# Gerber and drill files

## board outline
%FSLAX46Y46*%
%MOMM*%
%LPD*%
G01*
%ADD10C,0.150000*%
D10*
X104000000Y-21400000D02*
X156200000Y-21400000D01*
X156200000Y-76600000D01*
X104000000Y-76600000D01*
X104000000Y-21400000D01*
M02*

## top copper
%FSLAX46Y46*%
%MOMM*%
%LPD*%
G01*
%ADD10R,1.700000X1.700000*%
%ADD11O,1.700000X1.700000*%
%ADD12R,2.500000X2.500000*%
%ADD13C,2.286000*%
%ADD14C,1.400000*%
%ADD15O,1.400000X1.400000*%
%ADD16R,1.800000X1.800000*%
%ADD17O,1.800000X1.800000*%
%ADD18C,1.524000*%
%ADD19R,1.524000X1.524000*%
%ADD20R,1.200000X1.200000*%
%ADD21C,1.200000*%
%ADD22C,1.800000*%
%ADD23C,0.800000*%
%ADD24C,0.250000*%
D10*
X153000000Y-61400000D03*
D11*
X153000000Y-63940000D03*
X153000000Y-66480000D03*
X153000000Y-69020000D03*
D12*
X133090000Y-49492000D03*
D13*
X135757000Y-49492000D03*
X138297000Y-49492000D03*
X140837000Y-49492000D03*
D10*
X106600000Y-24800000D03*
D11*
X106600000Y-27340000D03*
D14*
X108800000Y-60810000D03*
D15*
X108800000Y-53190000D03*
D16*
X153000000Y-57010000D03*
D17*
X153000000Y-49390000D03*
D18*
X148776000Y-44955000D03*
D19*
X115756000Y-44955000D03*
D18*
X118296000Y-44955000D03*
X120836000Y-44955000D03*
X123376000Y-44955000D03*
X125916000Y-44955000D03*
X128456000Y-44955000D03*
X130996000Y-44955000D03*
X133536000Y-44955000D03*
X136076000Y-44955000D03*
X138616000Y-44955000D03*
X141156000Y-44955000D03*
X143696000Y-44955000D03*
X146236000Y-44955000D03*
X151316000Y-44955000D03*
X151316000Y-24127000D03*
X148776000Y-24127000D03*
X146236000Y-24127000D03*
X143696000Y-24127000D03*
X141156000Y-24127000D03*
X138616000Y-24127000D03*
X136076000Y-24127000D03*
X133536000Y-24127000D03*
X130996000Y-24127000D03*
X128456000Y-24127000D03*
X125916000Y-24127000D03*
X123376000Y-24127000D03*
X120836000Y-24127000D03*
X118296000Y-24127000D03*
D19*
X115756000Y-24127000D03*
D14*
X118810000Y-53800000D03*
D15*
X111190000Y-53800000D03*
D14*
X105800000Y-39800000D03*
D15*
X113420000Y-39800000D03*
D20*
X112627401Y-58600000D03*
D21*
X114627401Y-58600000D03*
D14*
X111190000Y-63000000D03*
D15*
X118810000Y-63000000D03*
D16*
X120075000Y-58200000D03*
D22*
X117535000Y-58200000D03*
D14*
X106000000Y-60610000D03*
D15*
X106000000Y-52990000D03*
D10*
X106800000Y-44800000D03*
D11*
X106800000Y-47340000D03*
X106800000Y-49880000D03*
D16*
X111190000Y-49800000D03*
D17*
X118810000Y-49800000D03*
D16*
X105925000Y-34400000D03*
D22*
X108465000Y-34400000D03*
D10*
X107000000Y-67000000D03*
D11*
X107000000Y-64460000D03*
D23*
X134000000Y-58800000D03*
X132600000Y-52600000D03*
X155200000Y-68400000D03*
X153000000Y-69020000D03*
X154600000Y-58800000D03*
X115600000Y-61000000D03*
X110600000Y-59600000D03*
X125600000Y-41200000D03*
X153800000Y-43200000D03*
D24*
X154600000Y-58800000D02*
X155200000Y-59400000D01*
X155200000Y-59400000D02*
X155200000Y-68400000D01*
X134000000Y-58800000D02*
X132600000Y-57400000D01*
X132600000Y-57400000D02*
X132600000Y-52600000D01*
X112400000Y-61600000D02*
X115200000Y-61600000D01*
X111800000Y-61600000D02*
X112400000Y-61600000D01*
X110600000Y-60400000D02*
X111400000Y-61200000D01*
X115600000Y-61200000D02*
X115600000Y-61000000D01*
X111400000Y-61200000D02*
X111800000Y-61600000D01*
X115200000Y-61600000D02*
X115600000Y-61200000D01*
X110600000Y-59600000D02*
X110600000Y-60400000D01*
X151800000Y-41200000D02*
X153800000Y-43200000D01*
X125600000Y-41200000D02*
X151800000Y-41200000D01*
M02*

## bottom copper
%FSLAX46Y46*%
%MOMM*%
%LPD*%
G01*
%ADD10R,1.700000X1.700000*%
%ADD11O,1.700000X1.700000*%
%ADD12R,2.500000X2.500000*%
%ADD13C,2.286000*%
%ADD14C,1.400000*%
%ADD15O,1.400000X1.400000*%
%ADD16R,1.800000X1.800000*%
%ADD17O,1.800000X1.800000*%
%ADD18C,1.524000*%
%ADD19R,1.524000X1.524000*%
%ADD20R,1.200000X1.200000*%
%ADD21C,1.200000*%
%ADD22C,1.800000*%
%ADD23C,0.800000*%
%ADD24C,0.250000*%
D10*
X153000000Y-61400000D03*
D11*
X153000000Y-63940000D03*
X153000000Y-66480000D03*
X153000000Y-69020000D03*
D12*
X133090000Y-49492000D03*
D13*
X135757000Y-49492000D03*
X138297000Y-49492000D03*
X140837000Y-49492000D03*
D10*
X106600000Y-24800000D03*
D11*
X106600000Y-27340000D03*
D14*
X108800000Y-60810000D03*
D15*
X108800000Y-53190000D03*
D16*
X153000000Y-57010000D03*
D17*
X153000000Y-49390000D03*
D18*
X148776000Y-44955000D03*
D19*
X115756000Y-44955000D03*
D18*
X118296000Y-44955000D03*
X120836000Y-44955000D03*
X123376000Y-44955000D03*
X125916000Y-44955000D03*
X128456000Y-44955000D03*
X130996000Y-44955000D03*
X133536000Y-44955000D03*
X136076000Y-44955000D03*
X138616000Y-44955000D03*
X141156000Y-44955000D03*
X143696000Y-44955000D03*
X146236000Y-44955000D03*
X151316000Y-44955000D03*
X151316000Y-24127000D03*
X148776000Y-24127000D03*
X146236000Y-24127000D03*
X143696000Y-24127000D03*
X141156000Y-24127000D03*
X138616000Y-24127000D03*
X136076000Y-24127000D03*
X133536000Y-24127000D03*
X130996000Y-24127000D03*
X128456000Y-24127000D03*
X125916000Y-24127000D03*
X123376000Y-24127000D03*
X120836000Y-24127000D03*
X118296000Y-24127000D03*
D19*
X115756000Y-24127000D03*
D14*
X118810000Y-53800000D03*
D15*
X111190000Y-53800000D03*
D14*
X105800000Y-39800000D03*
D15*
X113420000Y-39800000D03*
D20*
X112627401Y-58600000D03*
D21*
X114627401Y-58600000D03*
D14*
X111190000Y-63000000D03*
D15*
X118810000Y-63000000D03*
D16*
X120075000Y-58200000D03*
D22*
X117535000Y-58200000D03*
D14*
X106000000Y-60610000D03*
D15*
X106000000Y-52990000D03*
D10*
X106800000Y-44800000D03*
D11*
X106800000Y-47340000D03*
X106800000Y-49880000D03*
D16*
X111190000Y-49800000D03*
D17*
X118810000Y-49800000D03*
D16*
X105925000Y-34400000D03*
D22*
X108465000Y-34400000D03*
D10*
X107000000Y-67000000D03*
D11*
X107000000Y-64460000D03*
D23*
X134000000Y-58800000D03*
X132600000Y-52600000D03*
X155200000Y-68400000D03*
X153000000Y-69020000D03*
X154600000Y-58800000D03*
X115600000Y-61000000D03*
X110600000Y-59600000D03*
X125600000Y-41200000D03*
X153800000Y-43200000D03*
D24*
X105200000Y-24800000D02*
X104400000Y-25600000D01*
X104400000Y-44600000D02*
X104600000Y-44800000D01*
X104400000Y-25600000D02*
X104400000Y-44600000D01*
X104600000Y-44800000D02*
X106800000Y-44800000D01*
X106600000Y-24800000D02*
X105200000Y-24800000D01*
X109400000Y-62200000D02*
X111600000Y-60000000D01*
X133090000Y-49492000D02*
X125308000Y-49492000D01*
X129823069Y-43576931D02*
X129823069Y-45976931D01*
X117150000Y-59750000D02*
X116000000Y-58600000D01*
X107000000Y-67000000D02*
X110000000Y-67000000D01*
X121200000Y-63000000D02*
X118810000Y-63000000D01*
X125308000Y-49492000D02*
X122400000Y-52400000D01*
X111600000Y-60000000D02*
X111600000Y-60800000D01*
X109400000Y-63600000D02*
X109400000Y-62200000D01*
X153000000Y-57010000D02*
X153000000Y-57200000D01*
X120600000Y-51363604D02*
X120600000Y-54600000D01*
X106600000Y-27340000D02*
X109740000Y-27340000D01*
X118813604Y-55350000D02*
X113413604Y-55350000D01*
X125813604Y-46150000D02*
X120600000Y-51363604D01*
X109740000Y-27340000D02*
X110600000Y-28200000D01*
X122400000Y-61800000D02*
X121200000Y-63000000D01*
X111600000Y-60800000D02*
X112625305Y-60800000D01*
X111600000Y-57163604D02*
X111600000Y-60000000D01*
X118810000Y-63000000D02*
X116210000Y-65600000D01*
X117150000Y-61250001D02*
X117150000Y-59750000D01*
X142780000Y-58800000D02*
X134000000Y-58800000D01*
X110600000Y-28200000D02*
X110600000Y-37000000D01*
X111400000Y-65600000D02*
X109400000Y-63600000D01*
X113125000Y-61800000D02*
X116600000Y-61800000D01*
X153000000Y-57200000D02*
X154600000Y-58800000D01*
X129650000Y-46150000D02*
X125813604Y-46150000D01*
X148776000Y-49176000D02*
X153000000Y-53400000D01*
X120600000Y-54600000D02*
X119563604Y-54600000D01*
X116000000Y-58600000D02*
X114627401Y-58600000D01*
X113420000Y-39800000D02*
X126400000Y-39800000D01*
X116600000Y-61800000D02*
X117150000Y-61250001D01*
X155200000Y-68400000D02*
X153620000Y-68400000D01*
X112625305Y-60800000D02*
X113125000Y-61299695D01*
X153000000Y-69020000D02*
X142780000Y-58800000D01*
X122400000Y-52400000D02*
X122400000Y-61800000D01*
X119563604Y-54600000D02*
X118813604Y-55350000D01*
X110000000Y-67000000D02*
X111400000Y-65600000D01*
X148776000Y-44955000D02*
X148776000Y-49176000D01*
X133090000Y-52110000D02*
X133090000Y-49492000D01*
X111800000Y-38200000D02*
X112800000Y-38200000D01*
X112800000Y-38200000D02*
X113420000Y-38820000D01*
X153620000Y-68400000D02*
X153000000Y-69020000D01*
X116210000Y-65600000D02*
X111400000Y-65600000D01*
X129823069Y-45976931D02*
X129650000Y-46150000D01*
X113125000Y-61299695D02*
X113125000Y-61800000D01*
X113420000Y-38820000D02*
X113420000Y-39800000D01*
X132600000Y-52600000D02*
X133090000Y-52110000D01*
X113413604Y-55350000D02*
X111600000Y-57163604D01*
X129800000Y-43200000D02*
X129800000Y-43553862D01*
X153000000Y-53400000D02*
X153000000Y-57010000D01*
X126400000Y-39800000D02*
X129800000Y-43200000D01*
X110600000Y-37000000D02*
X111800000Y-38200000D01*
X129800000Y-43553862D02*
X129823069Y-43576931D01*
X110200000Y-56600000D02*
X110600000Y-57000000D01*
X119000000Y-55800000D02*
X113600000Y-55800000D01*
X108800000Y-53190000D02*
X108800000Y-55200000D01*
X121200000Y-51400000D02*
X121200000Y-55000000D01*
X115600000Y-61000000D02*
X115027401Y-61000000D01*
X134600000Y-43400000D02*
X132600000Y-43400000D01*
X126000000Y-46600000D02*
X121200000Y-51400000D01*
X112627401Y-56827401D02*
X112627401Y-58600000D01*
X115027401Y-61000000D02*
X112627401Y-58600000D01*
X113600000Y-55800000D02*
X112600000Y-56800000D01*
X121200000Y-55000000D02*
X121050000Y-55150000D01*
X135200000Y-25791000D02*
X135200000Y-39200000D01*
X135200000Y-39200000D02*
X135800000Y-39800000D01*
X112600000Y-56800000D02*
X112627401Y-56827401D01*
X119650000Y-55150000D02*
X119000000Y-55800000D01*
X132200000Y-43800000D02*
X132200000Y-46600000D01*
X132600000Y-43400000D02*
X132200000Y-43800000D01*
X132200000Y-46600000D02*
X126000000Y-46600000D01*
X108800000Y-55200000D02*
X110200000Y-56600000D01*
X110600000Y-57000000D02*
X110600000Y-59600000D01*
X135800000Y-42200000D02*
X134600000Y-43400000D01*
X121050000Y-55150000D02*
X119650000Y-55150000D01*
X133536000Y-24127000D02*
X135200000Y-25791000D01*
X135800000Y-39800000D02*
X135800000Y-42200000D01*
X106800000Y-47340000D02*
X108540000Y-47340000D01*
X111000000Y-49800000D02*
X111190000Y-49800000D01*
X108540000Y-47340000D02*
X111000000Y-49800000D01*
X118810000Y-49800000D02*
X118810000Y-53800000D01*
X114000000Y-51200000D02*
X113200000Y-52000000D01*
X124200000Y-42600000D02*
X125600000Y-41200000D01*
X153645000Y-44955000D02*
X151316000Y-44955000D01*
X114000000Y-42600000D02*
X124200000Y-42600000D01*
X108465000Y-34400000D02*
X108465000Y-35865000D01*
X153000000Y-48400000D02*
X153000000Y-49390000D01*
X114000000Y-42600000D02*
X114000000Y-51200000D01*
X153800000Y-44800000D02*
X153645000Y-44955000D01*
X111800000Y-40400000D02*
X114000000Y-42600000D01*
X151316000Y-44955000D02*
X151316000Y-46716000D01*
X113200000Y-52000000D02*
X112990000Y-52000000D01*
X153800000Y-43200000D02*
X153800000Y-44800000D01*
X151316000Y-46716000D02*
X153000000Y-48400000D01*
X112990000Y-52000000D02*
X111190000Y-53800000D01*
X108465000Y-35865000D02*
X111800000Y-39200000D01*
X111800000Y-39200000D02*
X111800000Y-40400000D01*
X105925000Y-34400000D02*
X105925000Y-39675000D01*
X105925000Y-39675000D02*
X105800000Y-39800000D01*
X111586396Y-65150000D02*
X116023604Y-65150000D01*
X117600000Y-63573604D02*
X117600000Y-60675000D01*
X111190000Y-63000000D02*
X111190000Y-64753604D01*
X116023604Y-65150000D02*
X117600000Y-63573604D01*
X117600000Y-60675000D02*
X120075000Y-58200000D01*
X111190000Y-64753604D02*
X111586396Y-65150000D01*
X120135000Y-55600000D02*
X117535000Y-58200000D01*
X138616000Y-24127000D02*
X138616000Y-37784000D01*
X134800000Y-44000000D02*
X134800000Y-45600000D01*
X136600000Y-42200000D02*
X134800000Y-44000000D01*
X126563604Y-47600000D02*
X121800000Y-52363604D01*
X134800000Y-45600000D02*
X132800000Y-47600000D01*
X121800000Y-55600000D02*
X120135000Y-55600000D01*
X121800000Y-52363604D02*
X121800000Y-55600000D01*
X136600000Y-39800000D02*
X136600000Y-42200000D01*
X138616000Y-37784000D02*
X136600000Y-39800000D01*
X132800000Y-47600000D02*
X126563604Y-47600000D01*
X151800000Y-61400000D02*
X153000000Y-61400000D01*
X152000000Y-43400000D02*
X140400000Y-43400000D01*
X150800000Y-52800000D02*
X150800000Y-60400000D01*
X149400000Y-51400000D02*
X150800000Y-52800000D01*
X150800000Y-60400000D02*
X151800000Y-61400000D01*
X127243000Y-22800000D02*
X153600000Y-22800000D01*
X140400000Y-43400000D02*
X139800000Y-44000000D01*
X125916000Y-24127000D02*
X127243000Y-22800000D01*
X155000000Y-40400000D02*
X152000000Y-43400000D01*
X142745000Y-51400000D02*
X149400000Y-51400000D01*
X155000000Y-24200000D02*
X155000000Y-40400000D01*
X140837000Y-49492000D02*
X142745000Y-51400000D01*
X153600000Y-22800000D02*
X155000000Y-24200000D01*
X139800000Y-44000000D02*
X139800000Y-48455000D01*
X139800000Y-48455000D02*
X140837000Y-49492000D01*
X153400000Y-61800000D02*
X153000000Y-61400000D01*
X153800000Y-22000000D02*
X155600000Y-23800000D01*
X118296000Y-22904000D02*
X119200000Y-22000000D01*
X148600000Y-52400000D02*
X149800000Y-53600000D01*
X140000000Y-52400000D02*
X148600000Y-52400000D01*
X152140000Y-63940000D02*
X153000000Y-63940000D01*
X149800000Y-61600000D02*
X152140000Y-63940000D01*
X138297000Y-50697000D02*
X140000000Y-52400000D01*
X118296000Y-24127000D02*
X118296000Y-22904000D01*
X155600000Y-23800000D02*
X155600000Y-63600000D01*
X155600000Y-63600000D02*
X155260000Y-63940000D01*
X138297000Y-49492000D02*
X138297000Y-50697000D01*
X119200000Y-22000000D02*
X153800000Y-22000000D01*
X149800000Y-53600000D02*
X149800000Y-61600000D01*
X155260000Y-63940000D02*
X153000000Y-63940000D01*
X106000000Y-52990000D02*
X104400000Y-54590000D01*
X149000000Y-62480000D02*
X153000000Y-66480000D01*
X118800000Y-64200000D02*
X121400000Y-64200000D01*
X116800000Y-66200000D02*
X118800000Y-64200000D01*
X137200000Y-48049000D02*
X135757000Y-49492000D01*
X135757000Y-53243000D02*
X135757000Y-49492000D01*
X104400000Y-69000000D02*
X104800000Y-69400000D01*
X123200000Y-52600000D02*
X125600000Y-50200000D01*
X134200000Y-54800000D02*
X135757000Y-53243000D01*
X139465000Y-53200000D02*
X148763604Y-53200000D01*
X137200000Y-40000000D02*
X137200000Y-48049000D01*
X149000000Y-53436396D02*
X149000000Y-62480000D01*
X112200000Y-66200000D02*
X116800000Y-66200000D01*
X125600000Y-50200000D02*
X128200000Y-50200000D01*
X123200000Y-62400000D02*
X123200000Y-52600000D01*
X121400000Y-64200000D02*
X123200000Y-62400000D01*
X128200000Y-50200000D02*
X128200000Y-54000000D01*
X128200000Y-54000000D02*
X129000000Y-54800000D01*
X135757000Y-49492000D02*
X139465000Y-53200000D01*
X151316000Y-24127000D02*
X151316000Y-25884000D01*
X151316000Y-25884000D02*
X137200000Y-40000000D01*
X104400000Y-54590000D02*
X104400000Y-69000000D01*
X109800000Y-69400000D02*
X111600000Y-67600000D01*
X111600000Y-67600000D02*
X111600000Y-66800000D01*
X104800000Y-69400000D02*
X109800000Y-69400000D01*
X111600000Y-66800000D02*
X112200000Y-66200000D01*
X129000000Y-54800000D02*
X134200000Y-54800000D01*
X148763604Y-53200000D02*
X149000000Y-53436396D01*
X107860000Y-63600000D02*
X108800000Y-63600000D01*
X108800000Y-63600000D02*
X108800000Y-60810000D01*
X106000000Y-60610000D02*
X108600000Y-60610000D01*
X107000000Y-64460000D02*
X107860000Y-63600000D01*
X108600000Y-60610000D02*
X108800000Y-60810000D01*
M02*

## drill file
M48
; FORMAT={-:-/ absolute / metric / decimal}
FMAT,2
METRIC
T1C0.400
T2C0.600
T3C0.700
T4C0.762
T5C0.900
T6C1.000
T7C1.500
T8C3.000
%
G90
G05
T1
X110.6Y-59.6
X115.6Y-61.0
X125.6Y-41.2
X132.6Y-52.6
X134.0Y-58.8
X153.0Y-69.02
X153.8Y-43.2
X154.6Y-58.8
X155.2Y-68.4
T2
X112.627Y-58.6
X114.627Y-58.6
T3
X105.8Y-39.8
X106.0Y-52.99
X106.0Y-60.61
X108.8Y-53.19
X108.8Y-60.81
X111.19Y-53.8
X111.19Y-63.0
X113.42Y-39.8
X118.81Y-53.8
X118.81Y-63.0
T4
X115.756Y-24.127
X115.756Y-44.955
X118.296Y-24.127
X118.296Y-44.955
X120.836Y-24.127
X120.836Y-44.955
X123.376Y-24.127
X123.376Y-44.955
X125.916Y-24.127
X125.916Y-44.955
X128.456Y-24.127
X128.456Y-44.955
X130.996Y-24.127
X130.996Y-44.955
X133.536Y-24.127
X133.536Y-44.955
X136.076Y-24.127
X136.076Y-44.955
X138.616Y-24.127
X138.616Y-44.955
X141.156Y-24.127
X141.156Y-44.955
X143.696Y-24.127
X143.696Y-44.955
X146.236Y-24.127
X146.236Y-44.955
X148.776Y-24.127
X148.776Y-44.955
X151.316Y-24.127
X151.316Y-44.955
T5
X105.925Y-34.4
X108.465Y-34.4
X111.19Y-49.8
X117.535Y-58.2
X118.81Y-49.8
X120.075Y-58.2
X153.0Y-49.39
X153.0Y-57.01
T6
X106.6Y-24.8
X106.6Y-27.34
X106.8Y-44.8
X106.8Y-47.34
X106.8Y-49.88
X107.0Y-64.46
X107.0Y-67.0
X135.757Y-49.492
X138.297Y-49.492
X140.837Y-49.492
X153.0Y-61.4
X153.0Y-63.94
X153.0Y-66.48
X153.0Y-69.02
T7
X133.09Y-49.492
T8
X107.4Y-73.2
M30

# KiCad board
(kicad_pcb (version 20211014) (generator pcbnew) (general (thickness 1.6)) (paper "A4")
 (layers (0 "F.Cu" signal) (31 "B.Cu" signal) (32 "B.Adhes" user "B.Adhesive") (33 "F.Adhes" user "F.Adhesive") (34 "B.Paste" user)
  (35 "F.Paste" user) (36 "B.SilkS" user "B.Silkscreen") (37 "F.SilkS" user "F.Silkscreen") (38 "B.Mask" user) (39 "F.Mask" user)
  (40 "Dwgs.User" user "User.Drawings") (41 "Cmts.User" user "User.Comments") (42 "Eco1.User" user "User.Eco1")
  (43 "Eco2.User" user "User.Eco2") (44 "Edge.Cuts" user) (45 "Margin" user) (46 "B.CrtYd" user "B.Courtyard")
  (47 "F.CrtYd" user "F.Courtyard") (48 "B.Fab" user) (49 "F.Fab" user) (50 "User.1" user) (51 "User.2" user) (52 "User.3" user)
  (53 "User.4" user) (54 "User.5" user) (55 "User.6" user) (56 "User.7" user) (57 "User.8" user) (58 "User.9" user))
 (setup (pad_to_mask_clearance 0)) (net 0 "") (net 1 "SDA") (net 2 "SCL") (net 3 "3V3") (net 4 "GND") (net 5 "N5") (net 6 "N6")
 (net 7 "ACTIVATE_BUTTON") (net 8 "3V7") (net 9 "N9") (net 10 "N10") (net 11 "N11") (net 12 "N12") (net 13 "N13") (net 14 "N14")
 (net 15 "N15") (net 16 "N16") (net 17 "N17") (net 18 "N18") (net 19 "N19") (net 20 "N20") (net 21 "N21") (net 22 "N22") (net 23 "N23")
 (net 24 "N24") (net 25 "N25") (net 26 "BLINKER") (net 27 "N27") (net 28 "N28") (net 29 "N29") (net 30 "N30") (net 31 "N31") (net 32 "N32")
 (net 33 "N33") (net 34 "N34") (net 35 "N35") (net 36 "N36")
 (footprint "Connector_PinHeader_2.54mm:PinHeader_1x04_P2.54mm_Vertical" (layer "F.Cu") (at 153 61.4)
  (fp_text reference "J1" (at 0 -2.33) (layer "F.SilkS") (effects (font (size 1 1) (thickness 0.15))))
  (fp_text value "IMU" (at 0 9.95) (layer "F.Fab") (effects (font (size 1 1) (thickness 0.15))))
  (pad "1" thru_hole rect (at 0 0) (size 1.7 1.7) (drill 1) (layers *.Cu *.Mask) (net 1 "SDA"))
  (pad "2" thru_hole oval (at 0 2.54) (size 1.7 1.7) (drill 1) (layers *.Cu *.Mask) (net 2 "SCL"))
  (pad "3" thru_hole oval (at 0 5.08) (size 1.7 1.7) (drill 1) (layers *.Cu *.Mask) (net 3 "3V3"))
  (pad "4" thru_hole oval (at 0 7.62) (size 1.7 1.7) (drill 1) (layers *.Cu *.Mask) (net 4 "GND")))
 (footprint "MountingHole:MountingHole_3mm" (layer "F.Cu") (at 107.4 73.2)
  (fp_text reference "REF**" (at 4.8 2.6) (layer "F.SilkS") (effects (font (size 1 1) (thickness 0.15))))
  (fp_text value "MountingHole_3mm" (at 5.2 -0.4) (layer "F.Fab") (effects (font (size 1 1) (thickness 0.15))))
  (pad "" np_thru_hole circle (at 0 0) (size 3 3) (drill 3) (layers *.Cu *.Mask)))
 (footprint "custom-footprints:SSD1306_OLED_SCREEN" (layer "F.Cu") (at 122.295 48.095)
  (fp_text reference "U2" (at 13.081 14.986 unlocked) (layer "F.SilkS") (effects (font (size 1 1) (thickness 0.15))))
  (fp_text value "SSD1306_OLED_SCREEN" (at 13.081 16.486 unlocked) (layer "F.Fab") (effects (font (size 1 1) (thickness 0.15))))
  (pad "1" thru_hole rect (at 10.795 1.397) (size 2.5 2.5) (drill 1.5) (layers *.Cu *.Mask) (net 4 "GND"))
  (pad "2" thru_hole circle (at 13.462 1.397) (size 2.286 2.286) (drill 1) (layers *.Cu *.Mask) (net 3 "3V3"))
  (pad "3" thru_hole circle (at 16.002 1.397) (size 2.286 2.286) (drill 1) (layers *.Cu *.Mask) (remove_unused_layers) (keep_end_layers)
   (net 2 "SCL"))
  (pad "4" thru_hole circle (at 18.542 1.397) (size 2.286 2.286) (drill 1) (layers *.Cu *.Mask) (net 1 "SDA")))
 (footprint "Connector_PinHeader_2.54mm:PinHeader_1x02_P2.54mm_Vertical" (layer "F.Cu") (at 106.6 24.8)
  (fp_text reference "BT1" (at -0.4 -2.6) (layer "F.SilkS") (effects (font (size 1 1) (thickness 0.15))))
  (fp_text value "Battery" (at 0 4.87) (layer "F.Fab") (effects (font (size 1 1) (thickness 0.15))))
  (pad "1" thru_hole rect (at 0 0) (size 1.7 1.7) (drill 1) (layers *.Cu *.Mask) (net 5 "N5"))
  (pad "2" thru_hole oval (at 0 2.54) (size 1.7 1.7) (drill 1) (layers *.Cu *.Mask) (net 4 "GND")))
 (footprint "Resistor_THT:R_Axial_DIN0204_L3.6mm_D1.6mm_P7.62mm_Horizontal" (layer "F.Cu") (at 108.8 60.81 90)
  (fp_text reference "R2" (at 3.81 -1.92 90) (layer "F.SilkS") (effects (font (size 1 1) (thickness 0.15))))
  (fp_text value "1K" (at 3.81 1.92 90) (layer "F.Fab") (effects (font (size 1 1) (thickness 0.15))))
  (pad "1" thru_hole circle (at 0 0 90) (size 1.4 1.4) (drill 0.7) (layers *.Cu *.Mask) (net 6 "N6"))
  (pad "2" thru_hole oval (at 7.62 0 90) (size 1.4 1.4) (drill 0.7) (layers *.Cu *.Mask) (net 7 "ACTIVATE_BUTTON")))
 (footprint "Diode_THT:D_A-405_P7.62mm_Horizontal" (layer "F.Cu") (at 153 57.01 90)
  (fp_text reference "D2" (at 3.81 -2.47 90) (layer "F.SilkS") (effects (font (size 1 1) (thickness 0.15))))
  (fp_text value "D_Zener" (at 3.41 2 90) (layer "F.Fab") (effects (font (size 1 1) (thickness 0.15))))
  (pad "1" thru_hole rect (at 0 0 90) (size 1.8 1.8) (drill 0.9) (layers *.Cu *.Mask) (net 4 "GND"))
  (pad "2" thru_hole oval (at 7.62 0 90) (size 1.8 1.8) (drill 0.9) (layers *.Cu *.Mask) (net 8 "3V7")))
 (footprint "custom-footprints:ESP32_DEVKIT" (layer "F.Cu") (at 110.295 46.225 90)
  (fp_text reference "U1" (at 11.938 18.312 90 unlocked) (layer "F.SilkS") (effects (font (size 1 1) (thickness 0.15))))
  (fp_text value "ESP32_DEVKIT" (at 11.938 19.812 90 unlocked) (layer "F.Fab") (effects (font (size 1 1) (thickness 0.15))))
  (pad "1" thru_hole circle (at 1.27 38.481 90) (size 1.524 1.524) (drill 0.762) (layers *.Cu *.Mask) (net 4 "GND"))
  (pad "2" thru_hole rect (at 1.27 5.461 90) (size 1.524 1.524) (drill oval 0.762) (layers *.Cu *.Mask) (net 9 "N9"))
  (pad "3" thru_hole circle (at 1.27 8.001 90) (size 1.524 1.524) (drill 0.762) (layers *.Cu *.Mask) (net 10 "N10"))
  (pad "4" thru_hole circle (at 1.27 10.541 90) (size 1.524 1.524) (drill 0.762) (layers *.Cu *.Mask) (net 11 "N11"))
  (pad "5" thru_hole circle (at 1.27 13.081 90) (size 1.524 1.524) (drill 0.762) (layers *.Cu *.Mask) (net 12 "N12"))
  (pad "6" thru_hole circle (at 1.27 15.621 90) (size 1.524 1.524) (drill 0.762) (layers *.Cu *.Mask) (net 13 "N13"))
  (pad "7" thru_hole circle (at 1.27 18.161 90) (size 1.524 1.524) (drill 0.762) (layers *.Cu *.Mask) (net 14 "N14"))
  (pad "8" thru_hole circle (at 1.27 20.701 90) (size 1.524 1.524) (drill 0.762) (layers *.Cu *.Mask) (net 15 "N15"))
  (pad "9" thru_hole circle (at 1.27 23.241 90) (size 1.524 1.524) (drill 0.762) (layers *.Cu *.Mask) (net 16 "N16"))
  (pad "10" thru_hole circle (at 1.27 25.781 90) (size 1.524 1.524) (drill 0.762) (layers *.Cu *.Mask) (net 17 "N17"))
  (pad "11" thru_hole circle (at 1.27 28.321 90) (size 1.524 1.524) (drill 0.762) (layers *.Cu *.Mask) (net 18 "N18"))
  (pad "12" thru_hole circle (at 1.27 30.861 90) (size 1.524 1.524) (drill 0.762) (layers *.Cu *.Mask) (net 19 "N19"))
  (pad "13" thru_hole circle (at 1.27 33.401 90) (size 1.524 1.524) (drill 0.762) (layers *.Cu *.Mask) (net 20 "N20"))
  (pad "14" thru_hole circle (at 1.27 35.941 90) (size 1.524 1.524) (drill 0.762) (layers *.Cu *.Mask) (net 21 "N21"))
  (pad "16" thru_hole circle (at 1.27 41.021 90) (size 1.524 1.524) (drill 0.762) (layers *.Cu *.Mask) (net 8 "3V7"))
  (pad "24" thru_hole circle (at 22.098 41.021 90) (size 1.524 1.524) (drill 0.762) (layers *.Cu *.Mask) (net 3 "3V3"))
  (pad "25" thru_hole circle (at 22.098 38.481 90) (size 1.524 1.524) (drill 0.762) (layers *.Cu *.Mask) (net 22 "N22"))
  (pad "26" thru_hole circle (at 22.098 35.941 90) (size 1.524 1.524) (drill 0.762) (layers *.Cu *.Mask) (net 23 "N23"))
  (pad "27" thru_hole circle (at 22.098 33.401 90) (size 1.524 1.524) (drill 0.762) (layers *.Cu *.Mask) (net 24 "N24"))
  (pad "28" thru_hole circle (at 22.098 30.861 90) (size 1.524 1.524) (drill 0.762) (layers *.Cu *.Mask) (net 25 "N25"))
  (pad "29" thru_hole circle (at 22.098 28.321 90) (size 1.524 1.524) (drill 0.762) (layers *.Cu *.Mask) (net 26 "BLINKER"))
  (pad "30" thru_hole circle (at 22.098 25.781 90) (size 1.524 1.524) (drill 0.762) (layers *.Cu *.Mask) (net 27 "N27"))
  (pad "31" thru_hole circle (at 22.098 23.241 90) (size 1.524 1.524) (drill 0.762) (layers *.Cu *.Mask) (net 7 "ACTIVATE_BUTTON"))
  (pad "32" thru_hole circle (at 22.098 20.701 90) (size 1.524 1.524) (drill 0.762) (layers *.Cu *.Mask) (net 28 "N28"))
  (pad "33" thru_hole circle (at 22.098 18.161 90) (size 1.524 1.524) (drill 0.762) (layers *.Cu *.Mask) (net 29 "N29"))
  (pad "34" thru_hole circle (at 22.098 15.621 90) (size 1.524 1.524) (drill 0.762) (layers *.Cu *.Mask) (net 1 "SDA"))
  (pad "35" thru_hole circle (at 22.098 13.081 90) (size 1.524 1.524) (drill 0.762) (layers *.Cu *.Mask) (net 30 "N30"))
  (pad "36" thru_hole circle (at 22.098 10.541 90) (size 1.524 1.524) (drill 0.762) (layers *.Cu *.Mask) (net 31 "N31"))
  (pad "37" thru_hole circle (at 22.098 8.001 90) (size 1.524 1.524) (drill 0.762) (layers *.Cu *.Mask) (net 2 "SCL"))
  (pad "38" thru_hole rect (at 22.098 5.461 90) (size 1.524 1.524) (drill 0.762) (layers *.Cu *.Mask) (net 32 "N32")))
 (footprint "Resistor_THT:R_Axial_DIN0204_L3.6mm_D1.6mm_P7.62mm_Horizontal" (layer "F.Cu") (at 118.81 53.8 180)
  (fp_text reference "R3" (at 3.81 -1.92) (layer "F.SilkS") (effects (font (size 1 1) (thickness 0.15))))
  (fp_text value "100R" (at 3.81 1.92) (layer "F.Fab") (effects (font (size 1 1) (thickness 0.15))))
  (pad "1" thru_hole circle (at 0 0 180) (size 1.4 1.4) (drill 0.7) (layers *.Cu *.Mask) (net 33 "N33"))
  (pad "2" thru_hole oval (at 7.62 0 180) (size 1.4 1.4) (drill 0.7) (layers *.Cu *.Mask) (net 8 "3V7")))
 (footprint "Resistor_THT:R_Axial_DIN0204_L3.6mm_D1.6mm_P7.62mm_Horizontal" (layer "F.Cu") (at 105.8 39.8)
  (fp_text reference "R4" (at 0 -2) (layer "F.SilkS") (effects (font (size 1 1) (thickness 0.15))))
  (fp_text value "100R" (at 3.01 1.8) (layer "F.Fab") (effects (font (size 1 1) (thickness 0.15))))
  (pad "1" thru_hole circle (at 0 0) (size 1.4 1.4) (drill 0.7) (layers *.Cu *.Mask) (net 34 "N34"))
  (pad "2" thru_hole oval (at 7.62 0) (size 1.4 1.4) (drill 0.7) (layers *.Cu *.Mask) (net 4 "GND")))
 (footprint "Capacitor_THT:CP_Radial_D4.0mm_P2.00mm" (layer "F.Cu") (at 112.627401 58.6)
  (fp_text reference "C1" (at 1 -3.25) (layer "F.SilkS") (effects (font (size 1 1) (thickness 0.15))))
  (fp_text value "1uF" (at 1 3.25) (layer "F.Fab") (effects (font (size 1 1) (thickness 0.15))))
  (pad "1" thru_hole rect (at 0 0) (size 1.2 1.2) (drill 0.6) (layers *.Cu *.Mask) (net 7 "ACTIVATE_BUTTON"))
  (pad "2" thru_hole circle (at 2 0) (size 1.2 1.2) (drill 0.6) (layers *.Cu *.Mask) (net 4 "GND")))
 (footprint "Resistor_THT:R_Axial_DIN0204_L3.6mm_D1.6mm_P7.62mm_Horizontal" (layer "F.Cu") (at 111.19 63)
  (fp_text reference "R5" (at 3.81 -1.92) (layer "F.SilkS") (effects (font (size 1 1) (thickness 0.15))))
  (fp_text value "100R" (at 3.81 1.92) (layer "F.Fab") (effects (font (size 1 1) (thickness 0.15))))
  (pad "1" thru_hole circle (at 0 0) (size 1.4 1.4) (drill 0.7) (layers *.Cu *.Mask) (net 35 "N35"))
  (pad "2" thru_hole oval (at 7.62 0) (size 1.4 1.4) (drill 0.7) (layers *.Cu *.Mask) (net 4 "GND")))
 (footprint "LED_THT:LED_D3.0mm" (layer "F.Cu") (at 120.075 58.2 180)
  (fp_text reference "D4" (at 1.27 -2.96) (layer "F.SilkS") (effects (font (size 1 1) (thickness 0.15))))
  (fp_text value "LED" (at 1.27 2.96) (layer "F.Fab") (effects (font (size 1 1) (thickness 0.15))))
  (pad "1" thru_hole rect (at 0 0 180) (size 1.8 1.8) (drill 0.9) (layers *.Cu *.Mask) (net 35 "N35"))
  (pad "2" thru_hole circle (at 2.54 0 180) (size 1.8 1.8) (drill 0.9) (layers *.Cu *.Mask) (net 26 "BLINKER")))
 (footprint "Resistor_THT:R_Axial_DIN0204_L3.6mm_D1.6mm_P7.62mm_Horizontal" (layer "F.Cu") (at 106 60.61 90)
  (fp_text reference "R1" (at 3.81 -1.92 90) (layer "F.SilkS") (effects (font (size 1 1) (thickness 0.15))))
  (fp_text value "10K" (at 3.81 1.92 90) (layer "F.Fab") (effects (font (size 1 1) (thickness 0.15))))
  (pad "1" thru_hole circle (at 0 0 90) (size 1.4 1.4) (drill 0.7) (layers *.Cu *.Mask) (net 6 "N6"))
  (pad "2" thru_hole oval (at 7.62 0 90) (size 1.4 1.4) (drill 0.7) (layers *.Cu *.Mask) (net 3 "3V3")))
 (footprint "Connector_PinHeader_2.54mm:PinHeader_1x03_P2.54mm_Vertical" (layer "F.Cu") (at 106.8 44.8)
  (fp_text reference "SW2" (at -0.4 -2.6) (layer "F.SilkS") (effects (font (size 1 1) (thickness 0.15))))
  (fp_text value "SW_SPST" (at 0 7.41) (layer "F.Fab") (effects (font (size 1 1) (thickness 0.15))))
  (pad "1" thru_hole rect (at 0 0) (size 1.7 1.7) (drill 1) (layers *.Cu *.Mask) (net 5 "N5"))
  (pad "2" thru_hole oval (at 0 2.54) (size 1.7 1.7) (drill 1) (layers *.Cu *.Mask) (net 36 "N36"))
  (pad "3" thru_hole oval (at 0 5.08) (size 1.7 1.7) (drill 1) (layers *.Cu *.Mask)))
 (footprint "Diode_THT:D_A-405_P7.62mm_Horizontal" (layer "F.Cu") (at 111.19 49.8)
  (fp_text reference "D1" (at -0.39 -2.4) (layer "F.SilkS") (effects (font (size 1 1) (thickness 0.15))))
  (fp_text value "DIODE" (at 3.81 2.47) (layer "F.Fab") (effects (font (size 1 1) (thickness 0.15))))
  (pad "1" thru_hole rect (at 0 0) (size 1.8 1.8) (drill 0.9) (layers *.Cu *.Mask) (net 36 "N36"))
  (pad "2" thru_hole oval (at 7.62 0) (size 1.8 1.8) (drill 0.9) (layers *.Cu *.Mask) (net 33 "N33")))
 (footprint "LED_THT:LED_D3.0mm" (layer "F.Cu") (at 105.925 34.4)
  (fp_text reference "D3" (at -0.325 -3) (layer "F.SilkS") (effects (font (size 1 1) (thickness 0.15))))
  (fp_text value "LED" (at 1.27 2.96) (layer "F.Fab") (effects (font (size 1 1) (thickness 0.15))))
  (pad "1" thru_hole rect (at 0 0) (size 1.8 1.8) (drill 0.9) (layers *.Cu *.Mask) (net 34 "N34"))
  (pad "2" thru_hole circle (at 2.54 0) (size 1.8 1.8) (drill 0.9) (layers *.Cu *.Mask) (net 8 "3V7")))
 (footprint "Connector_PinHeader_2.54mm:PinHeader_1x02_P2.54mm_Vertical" (layer "F.Cu") (at 107 67 180)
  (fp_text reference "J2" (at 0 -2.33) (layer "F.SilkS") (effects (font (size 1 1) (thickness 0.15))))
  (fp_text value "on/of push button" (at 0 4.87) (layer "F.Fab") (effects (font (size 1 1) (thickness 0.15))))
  (pad "1" thru_hole rect (at 0 0 180) (size 1.7 1.7) (drill 1) (layers *.Cu *.Mask) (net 4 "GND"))
  (pad "2" thru_hole oval (at 0 2.54 180) (size 1.7 1.7) (drill 1) (layers *.Cu *.Mask) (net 6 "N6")))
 (gr_rect (start 104 21.4) (end 156.2 76.6) (layer "Edge.Cuts") (width 0.15) (fill none))
 (segment (start 105.2 24.8) (end 104.4 25.6) (width 0.25) (layer "B.Cu") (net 5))
 (segment (start 104.4 44.6) (end 104.6 44.8) (width 0.25) (layer "B.Cu") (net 5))
 (segment (start 104.4 25.6) (end 104.4 44.6) (width 0.25) (layer "B.Cu") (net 5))
 (segment (start 104.6 44.8) (end 106.8 44.8) (width 0.25) (layer "B.Cu") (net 5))
 (segment (start 106.6 24.8) (end 105.2 24.8) (width 0.25) (layer "B.Cu") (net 5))
 (segment (start 154.6 58.8) (end 155.2 59.4) (width 0.25) (layer "F.Cu") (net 4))
 (segment (start 155.2 59.4) (end 155.2 68.4) (width 0.25) (layer "F.Cu") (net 4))
 (segment (start 134 58.8) (end 132.6 57.4) (width 0.25) (layer "F.Cu") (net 4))
 (segment (start 132.6 57.4) (end 132.6 52.6) (width 0.25) (layer "F.Cu") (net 4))
 (via (at 134 58.8) (size 0.8) (drill 0.4) (layers "F.Cu" "B.Cu") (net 4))
 (via (at 132.6 52.6) (size 0.8) (drill 0.4) (layers "F.Cu" "B.Cu") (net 4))
 (via (at 155.2 68.4) (size 0.8) (drill 0.4) (layers "F.Cu" "B.Cu") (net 4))
 (via (at 153 69.02) (size 0.8) (drill 0.4) (layers "F.Cu" "B.Cu") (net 4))
 (via (at 154.6 58.8) (size 0.8) (drill 0.4) (layers "F.Cu" "B.Cu") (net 4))
 (segment (start 109.4 62.2) (end 111.6 60) (width 0.25) (layer "B.Cu") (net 4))
 (segment (start 133.09 49.492) (end 125.308 49.492) (width 0.25) (layer "B.Cu") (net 4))
 (segment (start 129.823069 43.576931) (end 129.823069 45.976931) (width 0.25) (layer "B.Cu") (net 4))
 (segment (start 117.15 59.75) (end 116 58.6) (width 0.25) (layer "B.Cu") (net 4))
 (segment (start 107 67) (end 110 67) (width 0.25) (layer "B.Cu") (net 4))
 (segment (start 121.2 63) (end 118.81 63) (width 0.25) (layer "B.Cu") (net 4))
 (segment (start 125.308 49.492) (end 122.4 52.4) (width 0.25) (layer "B.Cu") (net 4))
 (segment (start 111.6 60) (end 111.6 60.8) (width 0.25) (layer "B.Cu") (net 4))
 (segment (start 109.4 63.6) (end 109.4 62.2) (width 0.25) (layer "B.Cu") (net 4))
 (segment (start 153 57.01) (end 153 57.2) (width 0.25) (layer "B.Cu") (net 4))
 (segment (start 120.6 51.363604) (end 120.6 54.6) (width 0.25) (layer "B.Cu") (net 4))
 (segment (start 106.6 27.34) (end 109.74 27.34) (width 0.25) (layer "B.Cu") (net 4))
 (segment (start 118.813604 55.35) (end 113.413604 55.35) (width 0.25) (layer "B.Cu") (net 4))
 (segment (start 125.813604 46.15) (end 120.6 51.363604) (width 0.25) (layer "B.Cu") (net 4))
 (segment (start 109.74 27.34) (end 110.6 28.2) (width 0.25) (layer "B.Cu") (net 4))
 (segment (start 122.4 61.8) (end 121.2 63) (width 0.25) (layer "B.Cu") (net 4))
 (segment (start 111.6 60.8) (end 112.625305 60.8) (width 0.25) (layer "B.Cu") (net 4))
 (segment (start 111.6 57.163604) (end 111.6 60) (width 0.25) (layer "B.Cu") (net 4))
 (segment (start 118.81 63) (end 116.21 65.6) (width 0.25) (layer "B.Cu") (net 4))
 (segment (start 117.15 61.250001) (end 117.15 59.75) (width 0.25) (layer "B.Cu") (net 4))
 (segment (start 142.78 58.8) (end 134 58.8) (width 0.25) (layer "B.Cu") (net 4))
 (segment (start 110.6 28.2) (end 110.6 37) (width 0.25) (layer "B.Cu") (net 4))
 (segment (start 111.4 65.6) (end 109.4 63.6) (width 0.25) (layer "B.Cu") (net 4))
 (segment (start 113.125 61.8) (end 116.6 61.8) (width 0.25) (layer "B.Cu") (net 4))
 (segment (start 153 57.2) (end 154.6 58.8) (width 0.25) (layer "B.Cu") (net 4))
 (segment (start 129.65 46.15) (end 125.813604 46.15) (width 0.25) (layer "B.Cu") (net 4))
 (segment (start 148.776 49.176) (end 153 53.4) (width 0.25) (layer "B.Cu") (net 4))
 (segment (start 120.6 54.6) (end 119.563604 54.6) (width 0.25) (layer "B.Cu") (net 4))
 (segment (start 116 58.6) (end 114.627401 58.6) (width 0.25) (layer "B.Cu") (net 4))
 (segment (start 113.42 39.8) (end 126.4 39.8) (width 0.25) (layer "B.Cu") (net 4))
 (segment (start 116.6 61.8) (end 117.15 61.250001) (width 0.25) (layer "B.Cu") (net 4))
 (segment (start 155.2 68.4) (end 153.62 68.4) (width 0.25) (layer "B.Cu") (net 4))
 (segment (start 112.625305 60.8) (end 113.125 61.299695) (width 0.25) (layer "B.Cu") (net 4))
 (segment (start 153 69.02) (end 142.78 58.8) (width 0.25) (layer "B.Cu") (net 4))
 (segment (start 122.4 52.4) (end 122.4 61.8) (width 0.25) (layer "B.Cu") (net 4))
 (segment (start 119.563604 54.6) (end 118.813604 55.35) (width 0.25) (layer "B.Cu") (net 4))
 (segment (start 110 67) (end 111.4 65.6) (width 0.25) (layer "B.Cu") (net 4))
 (segment (start 148.776 44.955) (end 148.776 49.176) (width 0.25) (layer "B.Cu") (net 4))
 (segment (start 133.09 52.11) (end 133.09 49.492) (width 0.25) (layer "B.Cu") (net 4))
 (segment (start 111.8 38.2) (end 112.8 38.2) (width 0.25) (layer "B.Cu") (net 4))
 (segment (start 112.8 38.2) (end 113.42 38.82) (width 0.25) (layer "B.Cu") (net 4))
 (segment (start 153.62 68.4) (end 153 69.02) (width 0.25) (layer "B.Cu") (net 4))
 (segment (start 116.21 65.6) (end 111.4 65.6) (width 0.25) (layer "B.Cu") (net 4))
 (segment (start 129.823069 45.976931) (end 129.65 46.15) (width 0.25) (layer "B.Cu") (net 4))
 (segment (start 113.125 61.299695) (end 113.125 61.8) (width 0.25) (layer "B.Cu") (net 4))
 (segment (start 113.42 38.82) (end 113.42 39.8) (width 0.25) (layer "B.Cu") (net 4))
 (segment (start 132.6 52.6) (end 133.09 52.11) (width 0.25) (layer "B.Cu") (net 4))
 (segment (start 113.413604 55.35) (end 111.6 57.163604) (width 0.25) (layer "B.Cu") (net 4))
 (segment (start 129.8 43.2) (end 129.8 43.553862) (width 0.25) (layer "B.Cu") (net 4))
 (segment (start 153 53.4) (end 153 57.01) (width 0.25) (layer "B.Cu") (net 4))
 (segment (start 126.4 39.8) (end 129.8 43.2) (width 0.25) (layer "B.Cu") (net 4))
 (segment (start 110.6 37) (end 111.8 38.2) (width 0.25) (layer "B.Cu") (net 4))
 (segment (start 129.8 43.553862) (end 129.823069 43.576931) (width 0.25) (layer "B.Cu") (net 4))
 (segment (start 112.4 61.6) (end 115.2 61.6) (width 0.25) (layer "F.Cu") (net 7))
 (segment (start 111.8 61.6) (end 112.4 61.6) (width 0.25) (layer "F.Cu") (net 7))
 (segment (start 110.6 60.4) (end 111.4 61.2) (width 0.25) (layer "F.Cu") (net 7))
 (segment (start 115.6 61.2) (end 115.6 61) (width 0.25) (layer "F.Cu") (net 7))
 (segment (start 111.4 61.2) (end 111.8 61.6) (width 0.25) (layer "F.Cu") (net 7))
 (segment (start 115.2 61.6) (end 115.6 61.2) (width 0.25) (layer "F.Cu") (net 7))
 (segment (start 110.6 59.6) (end 110.6 60.4) (width 0.25) (layer "F.Cu") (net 7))
 (via (at 115.6 61) (size 0.8) (drill 0.4) (layers "F.Cu" "B.Cu") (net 7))
 (via (at 110.6 59.6) (size 0.8) (drill 0.4) (layers "F.Cu" "B.Cu") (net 7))
 (segment (start 110.2 56.6) (end 110.6 57) (width 0.25) (layer "B.Cu") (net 7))
 (segment (start 119 55.8) (end 113.6 55.8) (width 0.25) (layer "B.Cu") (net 7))
 (segment (start 108.8 53.19) (end 108.8 55.2) (width 0.25) (layer "B.Cu") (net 7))
 (segment (start 121.2 51.4) (end 121.2 55) (width 0.25) (layer "B.Cu") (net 7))
 (segment (start 115.6 61) (end 115.027401 61) (width 0.25) (layer "B.Cu") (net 7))
 (segment (start 134.6 43.4) (end 132.6 43.4) (width 0.25) (layer "B.Cu") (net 7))
 (segment (start 126 46.6) (end 121.2 51.4) (width 0.25) (layer "B.Cu") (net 7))
 (segment (start 112.627401 56.827401) (end 112.627401 58.6) (width 0.25) (layer "B.Cu") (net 7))
 (segment (start 115.027401 61) (end 112.627401 58.6) (width 0.25) (layer "B.Cu") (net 7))
 (segment (start 113.6 55.8) (end 112.6 56.8) (width 0.25) (layer "B.Cu") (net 7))
 (segment (start 121.2 55) (end 121.05 55.15) (width 0.25) (layer "B.Cu") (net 7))
 (segment (start 135.2 25.791) (end 135.2 39.2) (width 0.25) (layer "B.Cu") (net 7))
 (segment (start 135.2 39.2) (end 135.8 39.8) (width 0.25) (layer "B.Cu") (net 7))
 (segment (start 112.6 56.8) (end 112.627401 56.827401) (width 0.25) (layer "B.Cu") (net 7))
 (segment (start 119.65 55.15) (end 119 55.8) (width 0.25) (layer "B.Cu") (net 7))
 (segment (start 132.2 43.8) (end 132.2 46.6) (width 0.25) (layer "B.Cu") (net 7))
 (segment (start 132.6 43.4) (end 132.2 43.8) (width 0.25) (layer "B.Cu") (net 7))
 (segment (start 132.2 46.6) (end 126 46.6) (width 0.25) (layer "B.Cu") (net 7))
 (segment (start 108.8 55.2) (end 110.2 56.6) (width 0.25) (layer "B.Cu") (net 7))
 (segment (start 110.6 57) (end 110.6 59.6) (width 0.25) (layer "B.Cu") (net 7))
 (segment (start 135.8 42.2) (end 134.6 43.4) (width 0.25) (layer "B.Cu") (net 7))
 (segment (start 121.05 55.15) (end 119.65 55.15) (width 0.25) (layer "B.Cu") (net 7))
 (segment (start 133.536 24.127) (end 135.2 25.791) (width 0.25) (layer "B.Cu") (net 7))
 (segment (start 135.8 39.8) (end 135.8 42.2) (width 0.25) (layer "B.Cu") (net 7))
 (segment (start 106.8 47.34) (end 108.54 47.34) (width 0.25) (layer "B.Cu") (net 36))
 (segment (start 111 49.8) (end 111.19 49.8) (width 0.25) (layer "B.Cu") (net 36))
 (segment (start 108.54 47.34) (end 111 49.8) (width 0.25) (layer "B.Cu") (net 36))
 (segment (start 118.81 49.8) (end 118.81 53.8) (width 0.25) (layer "B.Cu") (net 33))
 (segment (start 151.8 41.2) (end 153.8 43.2) (width 0.25) (layer "F.Cu") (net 8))
 (segment (start 125.6 41.2) (end 151.8 41.2) (width 0.25) (layer "F.Cu") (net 8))
 (via (at 125.6 41.2) (size 0.8) (drill 0.4) (layers "F.Cu" "B.Cu") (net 8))
 (via (at 153.8 43.2) (size 0.8) (drill 0.4) (layers "F.Cu" "B.Cu") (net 8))
 (segment (start 114 51.2) (end 113.2 52) (width 0.25) (layer "B.Cu") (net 8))
 (segment (start 124.2 42.6) (end 125.6 41.2) (width 0.25) (layer "B.Cu") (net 8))
 (segment (start 153.645 44.955) (end 151.316 44.955) (width 0.25) (layer "B.Cu") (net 8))
 (segment (start 114 42.6) (end 124.2 42.6) (width 0.25) (layer "B.Cu") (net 8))
 (segment (start 108.465 34.4) (end 108.465 35.865) (width 0.25) (layer "B.Cu") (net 8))
 (segment (start 153 48.4) (end 153 49.39) (width 0.25) (layer "B.Cu") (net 8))
 (segment (start 114 42.6) (end 114 51.2) (width 0.25) (layer "B.Cu") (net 8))
 (segment (start 153.8 44.8) (end 153.645 44.955) (width 0.25) (layer "B.Cu") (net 8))
 (segment (start 111.8 40.4) (end 114 42.6) (width 0.25) (layer "B.Cu") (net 8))
 (segment (start 151.316 44.955) (end 151.316 46.716) (width 0.25) (layer "B.Cu") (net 8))
 (segment (start 113.2 52) (end 112.99 52) (width 0.25) (layer "B.Cu") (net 8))
 (segment (start 153.8 43.2) (end 153.8 44.8) (width 0.25) (layer "B.Cu") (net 8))
 (segment (start 151.316 46.716) (end 153 48.4) (width 0.25) (layer "B.Cu") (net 8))
 (segment (start 112.99 52) (end 111.19 53.8) (width 0.25) (layer "B.Cu") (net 8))
 (segment (start 108.465 35.865) (end 111.8 39.2) (width 0.25) (layer "B.Cu") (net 8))
 (segment (start 111.8 39.2) (end 111.8 40.4) (width 0.25) (layer "B.Cu") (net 8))
 (segment (start 105.925 34.4) (end 105.925 39.675) (width 0.25) (layer "B.Cu") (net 34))
 (segment (start 105.925 39.675) (end 105.8 39.8) (width 0.25) (layer "B.Cu") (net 34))
 (segment (start 111.586396 65.15) (end 116.023604 65.15) (width 0.25) (layer "B.Cu") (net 35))
 (segment (start 117.6 63.573604) (end 117.6 60.675) (width 0.25) (layer "B.Cu") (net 35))
 (segment (start 111.19 63) (end 111.19 64.753604) (width 0.25) (layer "B.Cu") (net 35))
 (segment (start 116.023604 65.15) (end 117.6 63.573604) (width 0.25) (layer "B.Cu") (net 35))
 (segment (start 117.6 60.675) (end 120.075 58.2) (width 0.25) (layer "B.Cu") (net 35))
 (segment (start 111.19 64.753604) (end 111.586396 65.15) (width 0.25) (layer "B.Cu") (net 35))
 (segment (start 120.135 55.6) (end 117.535 58.2) (width 0.25) (layer "B.Cu") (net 26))
 (segment (start 138.616 24.127) (end 138.616 37.784) (width 0.25) (layer "B.Cu") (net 26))
 (segment (start 134.8 44) (end 134.8 45.6) (width 0.25) (layer "B.Cu") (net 26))
 (segment (start 136.6 42.2) (end 134.8 44) (width 0.25) (layer "B.Cu") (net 26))
 (segment (start 126.563604 47.6) (end 121.8 52.363604) (width 0.25) (layer "B.Cu") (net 26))
 (segment (start 134.8 45.6) (end 132.8 47.6) (width 0.25) (layer "B.Cu") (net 26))
 (segment (start 121.8 55.6) (end 120.135 55.6) (width 0.25) (layer "B.Cu") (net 26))
 (segment (start 121.8 52.363604) (end 121.8 55.6) (width 0.25) (layer "B.Cu") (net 26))
 (segment (start 136.6 39.8) (end 136.6 42.2) (width 0.25) (layer "B.Cu") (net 26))
 (segment (start 138.616 37.784) (end 136.6 39.8) (width 0.25) (layer "B.Cu") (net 26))
 (segment (start 132.8 47.6) (end 126.563604 47.6) (width 0.25) (layer "B.Cu") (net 26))
 (segment (start 151.8 61.4) (end 153 61.4) (width 0.25) (layer "B.Cu") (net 1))
 (segment (start 152 43.4) (end 140.4 43.4) (width 0.25) (layer "B.Cu") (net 1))
 (segment (start 150.8 52.8) (end 150.8 60.4) (width 0.25) (layer "B.Cu") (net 1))
 (segment (start 149.4 51.4) (end 150.8 52.8) (width 0.25) (layer "B.Cu") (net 1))
 (segment (start 150.8 60.4) (end 151.8 61.4) (width 0.25) (layer "B.Cu") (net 1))
 (segment (start 127.243 22.8) (end 153.6 22.8) (width 0.25) (layer "B.Cu") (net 1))
 (segment (start 140.4 43.4) (end 139.8 44) (width 0.25) (layer "B.Cu") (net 1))
 (segment (start 125.916 24.127) (end 127.243 22.8) (width 0.25) (layer "B.Cu") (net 1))
 (segment (start 155 40.4) (end 152 43.4) (width 0.25) (layer "B.Cu") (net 1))
 (segment (start 142.745 51.4) (end 149.4 51.4) (width 0.25) (layer "B.Cu") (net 1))
 (segment (start 155 24.2) (end 155 40.4) (width 0.25) (layer "B.Cu") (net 1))
 (segment (start 140.837 49.492) (end 142.745 51.4) (width 0.25) (layer "B.Cu") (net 1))
 (segment (start 153.6 22.8) (end 155 24.2) (width 0.25) (layer "B.Cu") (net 1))
 (segment (start 139.8 44) (end 139.8 48.455) (width 0.25) (layer "B.Cu") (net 1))
 (segment (start 139.8 48.455) (end 140.837 49.492) (width 0.25) (layer "B.Cu") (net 1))
 (segment (start 153.4 61.8) (end 153 61.4) (width 0.25) (layer "B.Cu") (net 1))
 (segment (start 153.8 22) (end 155.6 23.8) (width 0.25) (layer "B.Cu") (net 2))
 (segment (start 118.296 22.904) (end 119.2 22) (width 0.25) (layer "B.Cu") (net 2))
 (segment (start 148.6 52.4) (end 149.8 53.6) (width 0.25) (layer "B.Cu") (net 2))
 (segment (start 140 52.4) (end 148.6 52.4) (width 0.25) (layer "B.Cu") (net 2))
 (segment (start 152.14 63.94) (end 153 63.94) (width 0.25) (layer "B.Cu") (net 2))
 (segment (start 149.8 61.6) (end 152.14 63.94) (width 0.25) (layer "B.Cu") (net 2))
 (segment (start 138.297 50.697) (end 140 52.4) (width 0.25) (layer "B.Cu") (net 2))
 (segment (start 118.296 24.127) (end 118.296 22.904) (width 0.25) (layer "B.Cu") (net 2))
 (segment (start 155.6 23.8) (end 155.6 63.6) (width 0.25) (layer "B.Cu") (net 2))
 (segment (start 155.6 63.6) (end 155.26 63.94) (width 0.25) (layer "B.Cu") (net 2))
 (segment (start 138.297 49.492) (end 138.297 50.697) (width 0.25) (layer "B.Cu") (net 2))
 (segment (start 119.2 22) (end 153.8 22) (width 0.25) (layer "B.Cu") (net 2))
 (segment (start 149.8 53.6) (end 149.8 61.6) (width 0.25) (layer "B.Cu") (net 2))
 (segment (start 155.26 63.94) (end 153 63.94) (width 0.25) (layer "B.Cu") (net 2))
 (segment (start 106 52.99) (end 104.4 54.59) (width 0.25) (layer "B.Cu") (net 3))
 (segment (start 149 62.48) (end 153 66.48) (width 0.25) (layer "B.Cu") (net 3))
 (segment (start 118.8 64.2) (end 121.4 64.2) (width 0.25) (layer "B.Cu") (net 3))
 (segment (start 116.8 66.2) (end 118.8 64.2) (width 0.25) (layer "B.Cu") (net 3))
 (segment (start 137.2 48.049) (end 135.757 49.492) (width 0.25) (layer "B.Cu") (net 3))
 (segment (start 135.757 53.243) (end 135.757 49.492) (width 0.25) (layer "B.Cu") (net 3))
 (segment (start 104.4 69) (end 104.8 69.4) (width 0.25) (layer "B.Cu") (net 3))
 (segment (start 123.2 52.6) (end 125.6 50.2) (width 0.25) (layer "B.Cu") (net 3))
 (segment (start 134.2 54.8) (end 135.757 53.243) (width 0.25) (layer "B.Cu") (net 3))
 (segment (start 139.465 53.2) (end 148.763604 53.2) (width 0.25) (layer "B.Cu") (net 3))
 (segment (start 137.2 40) (end 137.2 48.049) (width 0.25) (layer "B.Cu") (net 3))
 (segment (start 149 53.436396) (end 149 62.48) (width 0.25) (layer "B.Cu") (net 3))
 (segment (start 112.2 66.2) (end 116.8 66.2) (width 0.25) (layer "B.Cu") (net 3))
 (segment (start 125.6 50.2) (end 128.2 50.2) (width 0.25) (layer "B.Cu") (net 3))
 (segment (start 123.2 62.4) (end 123.2 52.6) (width 0.25) (layer "B.Cu") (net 3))
 (segment (start 121.4 64.2) (end 123.2 62.4) (width 0.25) (layer "B.Cu") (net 3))
 (segment (start 128.2 50.2) (end 128.2 54) (width 0.25) (layer "B.Cu") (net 3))
 (segment (start 128.2 54) (end 129 54.8) (width 0.25) (layer "B.Cu") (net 3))
 (segment (start 135.757 49.492) (end 139.465 53.2) (width 0.25) (layer "B.Cu") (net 3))
 (segment (start 151.316 24.127) (end 151.316 25.884) (width 0.25) (layer "B.Cu") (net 3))
 (segment (start 151.316 25.884) (end 137.2 40) (width 0.25) (layer "B.Cu") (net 3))
 (segment (start 104.4 54.59) (end 104.4 69) (width 0.25) (layer "B.Cu") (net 3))
 (segment (start 109.8 69.4) (end 111.6 67.6) (width 0.25) (layer "B.Cu") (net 3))
 (segment (start 111.6 67.6) (end 111.6 66.8) (width 0.25) (layer "B.Cu") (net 3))
 (segment (start 104.8 69.4) (end 109.8 69.4) (width 0.25) (layer "B.Cu") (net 3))
 (segment (start 111.6 66.8) (end 112.2 66.2) (width 0.25) (layer "B.Cu") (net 3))
 (segment (start 129 54.8) (end 134.2 54.8) (width 0.25) (layer "B.Cu") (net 3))
 (segment (start 148.763604 53.2) (end 149 53.436396) (width 0.25) (layer "B.Cu") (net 3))
 (segment (start 107.86 63.6) (end 108.8 63.6) (width 0.25) (layer "B.Cu") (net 6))
 (segment (start 108.8 63.6) (end 108.8 60.81) (width 0.25) (layer "B.Cu") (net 6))
 (segment (start 106 60.61) (end 108.6 60.61) (width 0.25) (layer "B.Cu") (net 6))
 (segment (start 107 64.46) (end 107.86 63.6) (width 0.25) (layer "B.Cu") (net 6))
 (segment (start 108.6 60.61) (end 108.8 60.81) (width 0.25) (layer "B.Cu") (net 6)))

